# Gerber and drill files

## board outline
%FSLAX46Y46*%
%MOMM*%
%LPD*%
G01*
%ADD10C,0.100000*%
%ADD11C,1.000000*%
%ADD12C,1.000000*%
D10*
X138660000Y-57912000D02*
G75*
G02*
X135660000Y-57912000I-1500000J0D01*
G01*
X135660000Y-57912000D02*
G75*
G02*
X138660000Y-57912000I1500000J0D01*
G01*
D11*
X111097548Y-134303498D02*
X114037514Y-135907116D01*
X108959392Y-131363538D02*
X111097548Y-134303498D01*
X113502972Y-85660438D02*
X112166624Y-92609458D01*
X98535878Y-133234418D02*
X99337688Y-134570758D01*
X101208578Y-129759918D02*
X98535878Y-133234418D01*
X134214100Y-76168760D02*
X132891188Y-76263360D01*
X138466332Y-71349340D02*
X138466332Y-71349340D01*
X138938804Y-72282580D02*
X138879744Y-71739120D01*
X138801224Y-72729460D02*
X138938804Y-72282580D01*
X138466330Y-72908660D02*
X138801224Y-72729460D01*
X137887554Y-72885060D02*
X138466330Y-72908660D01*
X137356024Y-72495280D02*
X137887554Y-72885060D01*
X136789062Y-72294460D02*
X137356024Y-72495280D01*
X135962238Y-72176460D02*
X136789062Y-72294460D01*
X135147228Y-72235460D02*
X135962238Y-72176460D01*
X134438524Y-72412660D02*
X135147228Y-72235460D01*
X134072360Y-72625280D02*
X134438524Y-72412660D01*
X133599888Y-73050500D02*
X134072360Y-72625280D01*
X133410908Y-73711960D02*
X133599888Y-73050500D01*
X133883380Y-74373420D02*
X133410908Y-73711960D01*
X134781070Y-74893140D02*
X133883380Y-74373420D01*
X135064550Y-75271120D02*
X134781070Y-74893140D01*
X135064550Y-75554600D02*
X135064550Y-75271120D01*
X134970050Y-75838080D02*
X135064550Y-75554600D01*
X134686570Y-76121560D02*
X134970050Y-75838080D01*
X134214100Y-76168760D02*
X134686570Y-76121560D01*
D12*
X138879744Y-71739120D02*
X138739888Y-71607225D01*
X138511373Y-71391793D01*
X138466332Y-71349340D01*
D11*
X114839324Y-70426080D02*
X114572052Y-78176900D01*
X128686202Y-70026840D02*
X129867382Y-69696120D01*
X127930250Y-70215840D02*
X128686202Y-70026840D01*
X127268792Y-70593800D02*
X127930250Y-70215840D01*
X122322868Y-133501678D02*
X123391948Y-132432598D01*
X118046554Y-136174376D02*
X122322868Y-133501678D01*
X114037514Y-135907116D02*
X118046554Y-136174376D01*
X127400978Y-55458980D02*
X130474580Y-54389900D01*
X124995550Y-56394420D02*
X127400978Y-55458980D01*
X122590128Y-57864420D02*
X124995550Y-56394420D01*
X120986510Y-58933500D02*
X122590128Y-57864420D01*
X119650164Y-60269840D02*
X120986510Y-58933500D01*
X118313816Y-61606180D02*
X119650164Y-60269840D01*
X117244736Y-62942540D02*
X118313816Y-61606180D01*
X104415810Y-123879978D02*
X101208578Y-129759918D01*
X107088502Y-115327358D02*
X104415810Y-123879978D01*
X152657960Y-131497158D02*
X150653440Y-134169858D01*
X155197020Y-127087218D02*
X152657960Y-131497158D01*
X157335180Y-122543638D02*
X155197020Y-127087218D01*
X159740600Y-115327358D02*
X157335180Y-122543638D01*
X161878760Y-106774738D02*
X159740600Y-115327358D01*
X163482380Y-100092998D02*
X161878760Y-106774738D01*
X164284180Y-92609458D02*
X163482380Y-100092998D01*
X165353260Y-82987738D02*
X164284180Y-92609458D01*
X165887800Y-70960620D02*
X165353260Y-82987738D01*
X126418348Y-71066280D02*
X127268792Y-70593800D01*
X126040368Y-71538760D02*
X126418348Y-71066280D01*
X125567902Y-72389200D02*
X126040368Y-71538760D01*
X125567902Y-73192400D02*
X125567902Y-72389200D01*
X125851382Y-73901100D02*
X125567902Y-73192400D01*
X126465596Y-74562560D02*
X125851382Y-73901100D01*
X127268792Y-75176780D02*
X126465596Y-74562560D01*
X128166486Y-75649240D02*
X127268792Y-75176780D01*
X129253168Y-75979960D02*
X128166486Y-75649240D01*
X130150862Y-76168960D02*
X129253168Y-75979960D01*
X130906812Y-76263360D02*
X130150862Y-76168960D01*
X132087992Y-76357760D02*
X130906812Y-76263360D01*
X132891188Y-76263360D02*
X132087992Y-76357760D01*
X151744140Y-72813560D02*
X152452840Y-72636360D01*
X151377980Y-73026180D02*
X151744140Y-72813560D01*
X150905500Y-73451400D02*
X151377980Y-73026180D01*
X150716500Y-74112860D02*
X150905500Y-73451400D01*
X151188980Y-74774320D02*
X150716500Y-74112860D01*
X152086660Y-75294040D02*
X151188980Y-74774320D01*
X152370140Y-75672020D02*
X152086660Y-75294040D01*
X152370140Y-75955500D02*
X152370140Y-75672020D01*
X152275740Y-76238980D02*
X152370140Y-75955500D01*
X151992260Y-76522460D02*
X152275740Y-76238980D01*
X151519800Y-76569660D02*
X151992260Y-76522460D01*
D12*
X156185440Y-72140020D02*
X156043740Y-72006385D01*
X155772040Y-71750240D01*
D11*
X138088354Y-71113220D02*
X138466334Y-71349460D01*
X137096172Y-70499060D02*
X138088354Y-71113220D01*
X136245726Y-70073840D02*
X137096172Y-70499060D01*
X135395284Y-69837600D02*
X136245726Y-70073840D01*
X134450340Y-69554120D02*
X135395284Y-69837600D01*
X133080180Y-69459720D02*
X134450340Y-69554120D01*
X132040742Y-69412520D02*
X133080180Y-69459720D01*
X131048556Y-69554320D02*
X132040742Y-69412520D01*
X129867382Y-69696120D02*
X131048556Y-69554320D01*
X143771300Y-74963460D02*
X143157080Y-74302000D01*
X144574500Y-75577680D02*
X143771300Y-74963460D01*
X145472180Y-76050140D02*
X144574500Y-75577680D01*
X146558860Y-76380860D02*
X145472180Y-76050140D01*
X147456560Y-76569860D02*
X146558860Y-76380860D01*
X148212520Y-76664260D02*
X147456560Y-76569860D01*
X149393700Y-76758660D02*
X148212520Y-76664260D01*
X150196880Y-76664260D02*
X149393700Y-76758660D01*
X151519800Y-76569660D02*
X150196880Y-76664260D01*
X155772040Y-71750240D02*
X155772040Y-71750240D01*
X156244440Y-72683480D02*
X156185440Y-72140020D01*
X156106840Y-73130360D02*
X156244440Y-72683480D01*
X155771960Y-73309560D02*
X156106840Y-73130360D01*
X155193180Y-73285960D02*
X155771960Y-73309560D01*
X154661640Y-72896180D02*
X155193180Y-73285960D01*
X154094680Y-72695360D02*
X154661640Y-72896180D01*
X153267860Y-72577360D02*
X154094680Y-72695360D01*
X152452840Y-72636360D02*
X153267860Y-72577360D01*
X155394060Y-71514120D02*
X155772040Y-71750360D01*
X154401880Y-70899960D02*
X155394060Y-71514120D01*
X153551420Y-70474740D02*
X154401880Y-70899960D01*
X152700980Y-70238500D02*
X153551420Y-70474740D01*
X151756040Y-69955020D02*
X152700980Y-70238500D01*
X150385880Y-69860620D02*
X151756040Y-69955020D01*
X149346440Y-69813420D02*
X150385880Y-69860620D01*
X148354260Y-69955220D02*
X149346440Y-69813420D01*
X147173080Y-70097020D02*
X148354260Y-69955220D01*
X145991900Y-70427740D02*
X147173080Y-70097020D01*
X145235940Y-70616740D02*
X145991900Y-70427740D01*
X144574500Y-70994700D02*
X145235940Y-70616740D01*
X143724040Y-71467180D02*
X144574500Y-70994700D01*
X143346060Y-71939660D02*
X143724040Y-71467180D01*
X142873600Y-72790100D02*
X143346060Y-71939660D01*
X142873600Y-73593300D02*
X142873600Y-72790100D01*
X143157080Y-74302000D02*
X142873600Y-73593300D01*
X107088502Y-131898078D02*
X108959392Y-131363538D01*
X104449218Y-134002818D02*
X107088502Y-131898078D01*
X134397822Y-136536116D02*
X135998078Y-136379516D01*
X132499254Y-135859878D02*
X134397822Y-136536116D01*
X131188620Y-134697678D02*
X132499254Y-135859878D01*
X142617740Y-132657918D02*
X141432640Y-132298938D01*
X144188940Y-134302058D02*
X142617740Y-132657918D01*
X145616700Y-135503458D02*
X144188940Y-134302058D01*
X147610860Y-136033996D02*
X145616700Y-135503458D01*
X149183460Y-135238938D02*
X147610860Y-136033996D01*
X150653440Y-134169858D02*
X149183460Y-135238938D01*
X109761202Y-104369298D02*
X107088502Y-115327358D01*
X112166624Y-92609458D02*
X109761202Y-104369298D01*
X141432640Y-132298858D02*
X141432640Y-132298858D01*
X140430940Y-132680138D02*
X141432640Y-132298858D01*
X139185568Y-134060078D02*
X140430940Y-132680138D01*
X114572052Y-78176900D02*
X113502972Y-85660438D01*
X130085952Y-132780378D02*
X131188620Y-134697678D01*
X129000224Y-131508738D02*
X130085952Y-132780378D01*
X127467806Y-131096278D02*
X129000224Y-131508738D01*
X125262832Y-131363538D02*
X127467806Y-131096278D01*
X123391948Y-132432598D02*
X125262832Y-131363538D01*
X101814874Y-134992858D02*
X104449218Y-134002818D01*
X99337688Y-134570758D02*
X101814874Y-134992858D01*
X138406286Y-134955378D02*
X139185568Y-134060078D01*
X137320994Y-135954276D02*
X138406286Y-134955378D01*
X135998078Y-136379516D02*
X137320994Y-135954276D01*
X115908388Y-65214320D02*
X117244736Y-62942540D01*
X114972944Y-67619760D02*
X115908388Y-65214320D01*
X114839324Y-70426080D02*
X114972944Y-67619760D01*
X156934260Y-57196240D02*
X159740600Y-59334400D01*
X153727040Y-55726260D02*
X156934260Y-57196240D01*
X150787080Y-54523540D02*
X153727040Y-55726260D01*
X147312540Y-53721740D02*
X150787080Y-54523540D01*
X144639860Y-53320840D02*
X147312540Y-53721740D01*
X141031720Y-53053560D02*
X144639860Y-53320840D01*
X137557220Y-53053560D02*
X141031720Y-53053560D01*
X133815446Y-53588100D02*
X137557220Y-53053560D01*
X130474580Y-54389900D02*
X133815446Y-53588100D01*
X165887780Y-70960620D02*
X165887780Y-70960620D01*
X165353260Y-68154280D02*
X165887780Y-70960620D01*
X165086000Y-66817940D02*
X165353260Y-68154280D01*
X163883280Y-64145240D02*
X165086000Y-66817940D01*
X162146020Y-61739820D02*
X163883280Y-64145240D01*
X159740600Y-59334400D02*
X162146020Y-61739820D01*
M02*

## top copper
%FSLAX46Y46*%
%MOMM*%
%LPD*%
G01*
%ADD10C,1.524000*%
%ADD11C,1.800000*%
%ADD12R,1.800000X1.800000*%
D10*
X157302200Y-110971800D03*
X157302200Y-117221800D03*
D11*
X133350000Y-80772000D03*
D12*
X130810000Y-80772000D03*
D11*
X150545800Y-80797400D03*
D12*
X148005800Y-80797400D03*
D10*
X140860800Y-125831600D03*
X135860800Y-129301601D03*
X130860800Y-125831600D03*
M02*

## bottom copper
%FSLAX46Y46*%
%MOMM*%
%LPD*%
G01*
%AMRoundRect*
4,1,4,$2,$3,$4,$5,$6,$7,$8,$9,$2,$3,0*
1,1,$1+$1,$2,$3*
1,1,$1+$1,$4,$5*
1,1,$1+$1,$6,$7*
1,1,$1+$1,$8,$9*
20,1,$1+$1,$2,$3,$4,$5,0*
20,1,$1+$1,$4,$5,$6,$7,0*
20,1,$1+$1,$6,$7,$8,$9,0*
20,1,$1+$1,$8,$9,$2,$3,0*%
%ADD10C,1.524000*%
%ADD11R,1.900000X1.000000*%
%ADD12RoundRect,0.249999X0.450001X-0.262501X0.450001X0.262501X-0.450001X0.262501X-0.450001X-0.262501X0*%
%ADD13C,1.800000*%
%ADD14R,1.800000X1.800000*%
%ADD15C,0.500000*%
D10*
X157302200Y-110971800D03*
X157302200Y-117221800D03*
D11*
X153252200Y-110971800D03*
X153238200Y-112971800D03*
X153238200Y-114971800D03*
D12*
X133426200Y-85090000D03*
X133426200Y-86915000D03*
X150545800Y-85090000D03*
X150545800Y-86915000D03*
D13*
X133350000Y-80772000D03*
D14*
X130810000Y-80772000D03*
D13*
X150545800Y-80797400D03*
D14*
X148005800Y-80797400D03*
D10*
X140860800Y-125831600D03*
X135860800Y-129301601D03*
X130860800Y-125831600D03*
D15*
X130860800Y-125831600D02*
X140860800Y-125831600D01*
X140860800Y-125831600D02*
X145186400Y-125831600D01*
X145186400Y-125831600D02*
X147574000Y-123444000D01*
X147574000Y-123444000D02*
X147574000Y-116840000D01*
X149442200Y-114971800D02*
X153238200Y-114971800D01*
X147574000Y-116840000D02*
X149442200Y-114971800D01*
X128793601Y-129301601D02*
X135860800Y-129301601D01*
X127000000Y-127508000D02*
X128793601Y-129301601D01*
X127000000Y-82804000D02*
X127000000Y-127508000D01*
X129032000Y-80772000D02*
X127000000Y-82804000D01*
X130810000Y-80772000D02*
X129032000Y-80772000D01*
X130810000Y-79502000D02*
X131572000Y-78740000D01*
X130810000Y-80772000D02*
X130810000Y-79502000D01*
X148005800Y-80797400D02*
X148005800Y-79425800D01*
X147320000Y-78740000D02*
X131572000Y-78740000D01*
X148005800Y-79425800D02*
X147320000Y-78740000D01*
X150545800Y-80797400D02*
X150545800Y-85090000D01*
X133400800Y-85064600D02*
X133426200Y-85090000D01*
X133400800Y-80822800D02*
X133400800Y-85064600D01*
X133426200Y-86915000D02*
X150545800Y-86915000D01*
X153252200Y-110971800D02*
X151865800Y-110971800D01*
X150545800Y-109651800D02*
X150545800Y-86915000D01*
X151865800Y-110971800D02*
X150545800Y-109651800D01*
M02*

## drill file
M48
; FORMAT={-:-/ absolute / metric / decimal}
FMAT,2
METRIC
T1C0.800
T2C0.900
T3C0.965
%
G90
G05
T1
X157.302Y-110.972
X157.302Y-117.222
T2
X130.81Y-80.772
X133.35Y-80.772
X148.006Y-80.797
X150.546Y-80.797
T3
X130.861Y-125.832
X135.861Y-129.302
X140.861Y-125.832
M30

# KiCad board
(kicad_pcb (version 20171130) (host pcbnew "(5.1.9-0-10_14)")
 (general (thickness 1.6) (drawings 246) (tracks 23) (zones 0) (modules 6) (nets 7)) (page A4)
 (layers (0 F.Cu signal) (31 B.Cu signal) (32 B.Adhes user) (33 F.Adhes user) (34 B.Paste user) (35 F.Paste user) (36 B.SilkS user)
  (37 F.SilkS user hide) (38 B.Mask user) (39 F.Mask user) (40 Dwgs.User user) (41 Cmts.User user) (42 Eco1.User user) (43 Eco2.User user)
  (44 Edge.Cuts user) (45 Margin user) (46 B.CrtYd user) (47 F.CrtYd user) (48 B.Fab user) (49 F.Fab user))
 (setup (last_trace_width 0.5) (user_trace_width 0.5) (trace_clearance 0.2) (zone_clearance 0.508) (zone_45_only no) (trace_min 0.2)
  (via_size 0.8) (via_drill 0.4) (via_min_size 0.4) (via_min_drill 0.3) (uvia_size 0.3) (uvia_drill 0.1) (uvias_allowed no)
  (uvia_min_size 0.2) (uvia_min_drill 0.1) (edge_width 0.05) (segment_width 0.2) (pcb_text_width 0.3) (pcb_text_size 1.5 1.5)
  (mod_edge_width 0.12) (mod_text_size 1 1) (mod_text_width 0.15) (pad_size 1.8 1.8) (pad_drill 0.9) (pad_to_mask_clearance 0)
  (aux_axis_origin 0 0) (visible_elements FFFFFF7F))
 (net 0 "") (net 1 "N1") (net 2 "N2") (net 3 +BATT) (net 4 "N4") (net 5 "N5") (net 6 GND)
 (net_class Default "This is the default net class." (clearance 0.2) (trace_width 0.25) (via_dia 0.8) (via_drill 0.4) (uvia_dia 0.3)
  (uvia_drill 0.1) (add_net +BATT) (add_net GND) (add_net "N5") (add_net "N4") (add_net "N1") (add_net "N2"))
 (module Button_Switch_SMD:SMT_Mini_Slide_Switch (layer B.Cu) (at 155.0162 114.0968 270)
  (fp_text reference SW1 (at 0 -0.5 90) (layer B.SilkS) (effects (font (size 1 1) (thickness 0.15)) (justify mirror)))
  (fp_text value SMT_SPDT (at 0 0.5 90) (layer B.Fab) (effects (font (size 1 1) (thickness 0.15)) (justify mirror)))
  (pad "" thru_hole circle (at -3.125 -2.286 270) (size 1.524 1.524) (drill 0.8) (layers *.Cu *.Mask))
  (pad "" thru_hole circle (at 3.125 -2.286 270) (size 1.524 1.524) (drill 0.8) (layers *.Cu *.Mask))
  (pad 1 smd rect (at -3.125 1.764 270) (size 1 1.9) (layers B.Cu B.Paste B.Mask) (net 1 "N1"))
  (pad 2 smd rect (at -1.125 1.778 270) (size 1 1.9) (layers B.Cu B.Paste B.Mask) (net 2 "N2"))
  (pad 3 smd rect (at 0.875 1.778 270) (size 1 1.9) (layers B.Cu B.Paste B.Mask) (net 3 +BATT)))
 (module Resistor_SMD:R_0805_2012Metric (layer B.Cu) (at 133.4262 86.0025 90)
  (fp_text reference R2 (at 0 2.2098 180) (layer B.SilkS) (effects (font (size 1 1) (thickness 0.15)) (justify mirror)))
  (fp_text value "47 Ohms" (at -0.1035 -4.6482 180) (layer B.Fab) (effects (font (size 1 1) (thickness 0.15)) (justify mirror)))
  (pad 2 smd roundrect (at 0.9125 0 90) (size 1.025 1.4) (layers B.Cu B.Paste B.Mask) (roundrect_rratio 0.2439014634146341) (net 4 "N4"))
  (pad 1 smd roundrect (at -0.9125 0 90) (size 1.025 1.4) (layers B.Cu B.Paste B.Mask) (roundrect_rratio 0.2439014634146341) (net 1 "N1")))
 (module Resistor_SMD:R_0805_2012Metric (layer B.Cu) (at 150.5458 86.0025 90)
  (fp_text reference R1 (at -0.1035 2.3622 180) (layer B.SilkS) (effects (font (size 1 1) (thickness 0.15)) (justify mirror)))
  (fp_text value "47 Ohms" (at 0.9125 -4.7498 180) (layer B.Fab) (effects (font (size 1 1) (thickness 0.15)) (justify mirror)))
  (pad 2 smd roundrect (at 0.9125 0 90) (size 1.025 1.4) (layers B.Cu B.Paste B.Mask) (roundrect_rratio 0.2439014634146341) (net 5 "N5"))
  (pad 1 smd roundrect (at -0.9125 0 90) (size 1.025 1.4) (layers B.Cu B.Paste B.Mask) (roundrect_rratio 0.2439014634146341) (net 1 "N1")))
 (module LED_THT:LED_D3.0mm (layer B.Cu) (at 130.81 80.772)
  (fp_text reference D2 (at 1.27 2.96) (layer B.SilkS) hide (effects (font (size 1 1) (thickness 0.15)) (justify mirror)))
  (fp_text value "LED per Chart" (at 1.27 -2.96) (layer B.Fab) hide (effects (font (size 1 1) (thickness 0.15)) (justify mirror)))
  (pad 2 thru_hole circle (at 2.54 0) (size 1.8 1.8) (drill 0.9) (layers *.Cu *.Mask) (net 4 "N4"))
  (pad 1 thru_hole rect (at 0 0) (size 1.8 1.8) (drill 0.9) (layers *.Cu *.Mask) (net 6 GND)))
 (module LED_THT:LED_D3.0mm (layer B.Cu) (at 148.0058 80.7974)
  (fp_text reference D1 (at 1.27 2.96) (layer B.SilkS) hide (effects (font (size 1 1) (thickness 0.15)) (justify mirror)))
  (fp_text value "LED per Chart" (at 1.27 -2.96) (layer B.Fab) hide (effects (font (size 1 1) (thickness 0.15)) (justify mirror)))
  (pad 2 thru_hole circle (at 2.54 0) (size 1.8 1.8) (drill 0.9) (layers *.Cu *.Mask) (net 5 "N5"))
  (pad 1 thru_hole rect (at 0 0) (size 1.8 1.8) (drill 0.9) (layers *.Cu *.Mask) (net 6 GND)))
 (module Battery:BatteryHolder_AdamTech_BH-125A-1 (layer B.Cu) (at 130.8608 125.8316)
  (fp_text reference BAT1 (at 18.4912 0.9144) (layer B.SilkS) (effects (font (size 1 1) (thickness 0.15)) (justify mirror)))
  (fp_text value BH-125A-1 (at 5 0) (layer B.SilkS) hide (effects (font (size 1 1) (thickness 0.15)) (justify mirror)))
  (pad POS2 thru_hole circle (at 10 0) (size 1.524 1.524) (drill 0.9652) (layers *.Cu *.Mask) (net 3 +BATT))
  (pad NEG thru_hole circle (at 5 3.470001) (size 1.524 1.524) (drill 0.9652) (layers *.Cu *.Mask) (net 6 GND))
  (pad POS1 thru_hole circle (at 0 0) (size 1.524 1.524) (drill 0.9652) (layers *.Cu *.Mask) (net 3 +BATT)))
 (gr_circle (center 137.16 57.912) (end 138.66 57.912) (layer Edge.Cuts) (width 0.1))
 (gr_line (start 111.097548 134.303498) (end 114.037514 135.907116) (layer Edge.Cuts) (width 1))
 (gr_line (start 108.959392 131.363538) (end 111.097548 134.303498) (layer Edge.Cuts) (width 1))
 (gr_line (start 113.502972 85.660438) (end 112.166624 92.609458) (layer Edge.Cuts) (width 1))
 (gr_line (start 98.535878 133.234418) (end 99.337688 134.570758) (layer Edge.Cuts) (width 1))
 (gr_line (start 101.208578 129.759918) (end 98.535878 133.234418) (layer Edge.Cuts) (width 1))
 (gr_line (start 134.2141 76.16876) (end 132.891188 76.26336) (layer Edge.Cuts) (width 1))
 (gr_line (start 138.466332 71.34934) (end 138.466332 71.34934) (layer Edge.Cuts) (width 1))
 (gr_line (start 138.938804 72.28258) (end 138.879744 71.73912) (layer Edge.Cuts) (width 1))
 (gr_line (start 138.801224 72.72946) (end 138.938804 72.28258) (layer Edge.Cuts) (width 1))
 (gr_line (start 138.46633 72.90866) (end 138.801224 72.72946) (layer Edge.Cuts) (width 1))
 (gr_line (start 137.887554 72.88506) (end 138.46633 72.90866) (layer Edge.Cuts) (width 1))
 (gr_line (start 137.356024 72.49528) (end 137.887554 72.88506) (layer Edge.Cuts) (width 1))
 (gr_line (start 136.789062 72.29446) (end 137.356024 72.49528) (layer Edge.Cuts) (width 1))
 (gr_line (start 135.962238 72.17646) (end 136.789062 72.29446) (layer Edge.Cuts) (width 1))
 (gr_line (start 135.147228 72.23546) (end 135.962238 72.17646) (layer Edge.Cuts) (width 1))
 (gr_line (start 134.438524 72.41266) (end 135.147228 72.23546) (layer Edge.Cuts) (width 1))
 (gr_line (start 134.07236 72.62528) (end 134.438524 72.41266) (layer Edge.Cuts) (width 1))
 (gr_line (start 133.599888 73.0505) (end 134.07236 72.62528) (layer Edge.Cuts) (width 1))
 (gr_line (start 133.410908 73.71196) (end 133.599888 73.0505) (layer Edge.Cuts) (width 1))
 (gr_line (start 133.88338 74.37342) (end 133.410908 73.71196) (layer Edge.Cuts) (width 1))
 (gr_line (start 134.78107 74.89314) (end 133.88338 74.37342) (layer Edge.Cuts) (width 1))
 (gr_line (start 135.06455 75.27112) (end 134.78107 74.89314) (layer Edge.Cuts) (width 1))
 (gr_line (start 135.06455 75.5546) (end 135.06455 75.27112) (layer Edge.Cuts) (width 1))
 (gr_line (start 134.97005 75.83808) (end 135.06455 75.5546) (layer Edge.Cuts) (width 1))
 (gr_line (start 134.68657 76.12156) (end 134.97005 75.83808) (layer Edge.Cuts) (width 1))
 (gr_line (start 134.2141 76.16876) (end 134.68657 76.12156) (layer Edge.Cuts) (width 1))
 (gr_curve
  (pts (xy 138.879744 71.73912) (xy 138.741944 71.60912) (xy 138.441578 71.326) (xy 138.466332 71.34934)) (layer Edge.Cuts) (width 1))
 (gr_line (start 114.839324 70.42608) (end 114.572052 78.1769) (layer Edge.Cuts) (width 1))
 (gr_line (start 128.686202 70.02684) (end 129.867382 69.69612) (layer Edge.Cuts) (width 1))
 (gr_line (start 127.93025 70.21584) (end 128.686202 70.02684) (layer Edge.Cuts) (width 1))
 (gr_line (start 127.268792 70.5938) (end 127.93025 70.21584) (layer Edge.Cuts) (width 1))
 (gr_line (start 122.322868 133.501678) (end 123.391948 132.432598) (layer Edge.Cuts) (width 1))
 (gr_line (start 118.046554 136.174376) (end 122.322868 133.501678) (layer Edge.Cuts) (width 1))
 (gr_line (start 114.037514 135.907116) (end 118.046554 136.174376) (layer Edge.Cuts) (width 1))
 (gr_line (start 127.400978 55.45898) (end 130.47458 54.3899) (layer Edge.Cuts) (width 1))
 (gr_line (start 124.99555 56.39442) (end 127.400978 55.45898) (layer Edge.Cuts) (width 1))
 (gr_line (start 122.590128 57.86442) (end 124.99555 56.39442) (layer Edge.Cuts) (width 1))
 (gr_line (start 120.98651 58.9335) (end 122.590128 57.86442) (layer Edge.Cuts) (width 1))
 (gr_line (start 119.650164 60.26984) (end 120.98651 58.9335) (layer Edge.Cuts) (width 1))
 (gr_line (start 118.313816 61.60618) (end 119.650164 60.26984) (layer Edge.Cuts) (width 1))
 (gr_line (start 117.244736 62.94254) (end 118.313816 61.60618) (layer Edge.Cuts) (width 1))
 (gr_line (start 104.41581 123.879978) (end 101.208578 129.759918) (layer Edge.Cuts) (width 1))
 (gr_line (start 107.088502 115.327358) (end 104.41581 123.879978) (layer Edge.Cuts) (width 1))
 (gr_line (start 152.65796 131.497158) (end 150.65344 134.169858) (layer Edge.Cuts) (width 1))
 (gr_line (start 155.19702 127.087218) (end 152.65796 131.497158) (layer Edge.Cuts) (width 1))
 (gr_line (start 157.33518 122.543638) (end 155.19702 127.087218) (layer Edge.Cuts) (width 1))
 (gr_line (start 159.7406 115.327358) (end 157.33518 122.543638) (layer Edge.Cuts) (width 1))
 (gr_line (start 161.87876 106.774738) (end 159.7406 115.327358) (layer Edge.Cuts) (width 1))
 (gr_line (start 163.48238 100.092998) (end 161.87876 106.774738) (layer Edge.Cuts) (width 1))
 (gr_line (start 164.28418 92.609458) (end 163.48238 100.092998) (layer Edge.Cuts) (width 1))
 (gr_line (start 165.35326 82.987738) (end 164.28418 92.609458) (layer Edge.Cuts) (width 1))
 (gr_line (start 165.8878 70.96062) (end 165.35326 82.987738) (layer Edge.Cuts) (width 1))
 (gr_line (start 126.418348 71.06628) (end 127.268792 70.5938) (layer Edge.Cuts) (width 1))
 (gr_line (start 126.040368 71.53876) (end 126.418348 71.06628) (layer Edge.Cuts) (width 1))
 (gr_line (start 125.567902 72.3892) (end 126.040368 71.53876) (layer Edge.Cuts) (width 1))
 (gr_line (start 125.567902 73.1924) (end 125.567902 72.3892) (layer Edge.Cuts) (width 1))
 (gr_line (start 125.851382 73.9011) (end 125.567902 73.1924) (layer Edge.Cuts) (width 1))
 (gr_line (start 126.465596 74.56256) (end 125.851382 73.9011) (layer Edge.Cuts) (width 1))
 (gr_line (start 127.268792 75.17678) (end 126.465596 74.56256) (layer Edge.Cuts) (width 1))
 (gr_line (start 128.166486 75.64924) (end 127.268792 75.17678) (layer Edge.Cuts) (width 1))
 (gr_line (start 129.253168 75.97996) (end 128.166486 75.64924) (layer Edge.Cuts) (width 1))
 (gr_line (start 130.150862 76.16896) (end 129.253168 75.97996) (layer Edge.Cuts) (width 1))
 (gr_line (start 130.906812 76.26336) (end 130.150862 76.16896) (layer Edge.Cuts) (width 1))
 (gr_line (start 132.087992 76.35776) (end 130.906812 76.26336) (layer Edge.Cuts) (width 1))
 (gr_line (start 132.891188 76.26336) (end 132.087992 76.35776) (layer Edge.Cuts) (width 1))
 (gr_line (start 151.74414 72.81356) (end 152.45284 72.63636) (layer Edge.Cuts) (width 1))
 (gr_line (start 151.37798 73.02618) (end 151.74414 72.81356) (layer Edge.Cuts) (width 1))
 (gr_line (start 150.9055 73.4514) (end 151.37798 73.02618) (layer Edge.Cuts) (width 1))
 (gr_line (start 150.7165 74.11286) (end 150.9055 73.4514) (layer Edge.Cuts) (width 1))
 (gr_line (start 151.18898 74.77432) (end 150.7165 74.11286) (layer Edge.Cuts) (width 1))
 (gr_line (start 152.08666 75.29404) (end 151.18898 74.77432) (layer Edge.Cuts) (width 1))
 (gr_line (start 152.37014 75.67202) (end 152.08666 75.29404) (layer Edge.Cuts) (width 1))
 (gr_line (start 152.37014 75.9555) (end 152.37014 75.67202) (layer Edge.Cuts) (width 1))
 (gr_line (start 152.27574 76.23898) (end 152.37014 75.9555) (layer Edge.Cuts) (width 1))
 (gr_line (start 151.99226 76.52246) (end 152.27574 76.23898) (layer Edge.Cuts) (width 1))
 (gr_line (start 151.5198 76.56966) (end 151.99226 76.52246) (layer Edge.Cuts) (width 1))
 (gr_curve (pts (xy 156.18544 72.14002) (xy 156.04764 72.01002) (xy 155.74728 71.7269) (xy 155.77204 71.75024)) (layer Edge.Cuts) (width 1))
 (gr_line (start 138.088354 71.11322) (end 138.466334 71.34946) (layer Edge.Cuts) (width 1))
 (gr_line (start 137.096172 70.49906) (end 138.088354 71.11322) (layer Edge.Cuts) (width 1))
 (gr_line (start 136.245726 70.07384) (end 137.096172 70.49906) (layer Edge.Cuts) (width 1))
 (gr_line (start 135.395284 69.8376) (end 136.245726 70.07384) (layer Edge.Cuts) (width 1))
 (gr_line (start 134.45034 69.55412) (end 135.395284 69.8376) (layer Edge.Cuts) (width 1))
 (gr_line (start 133.08018 69.45972) (end 134.45034 69.55412) (layer Edge.Cuts) (width 1))
 (gr_line (start 132.040742 69.41252) (end 133.08018 69.45972) (layer Edge.Cuts) (width 1))
 (gr_line (start 131.048556 69.55432) (end 132.040742 69.41252) (layer Edge.Cuts) (width 1))
 (gr_line (start 129.867382 69.69612) (end 131.048556 69.55432) (layer Edge.Cuts) (width 1))
 (gr_line (start 143.7713 74.96346) (end 143.15708 74.302) (layer Edge.Cuts) (width 1))
 (gr_line (start 144.5745 75.57768) (end 143.7713 74.96346) (layer Edge.Cuts) (width 1))
 (gr_line (start 145.47218 76.05014) (end 144.5745 75.57768) (layer Edge.Cuts) (width 1))
 (gr_line (start 146.55886 76.38086) (end 145.47218 76.05014) (layer Edge.Cuts) (width 1))
 (gr_line (start 147.45656 76.56986) (end 146.55886 76.38086) (layer Edge.Cuts) (width 1))
 (gr_line (start 148.21252 76.66426) (end 147.45656 76.56986) (layer Edge.Cuts) (width 1))
 (gr_line (start 149.3937 76.75866) (end 148.21252 76.66426) (layer Edge.Cuts) (width 1))
 (gr_line (start 150.19688 76.66426) (end 149.3937 76.75866) (layer Edge.Cuts) (width 1))
 (gr_line (start 151.5198 76.56966) (end 150.19688 76.66426) (layer Edge.Cuts) (width 1))
 (gr_line (start 155.77204 71.75024) (end 155.77204 71.75024) (layer Edge.Cuts) (width 1))
 (gr_line (start 156.24444 72.68348) (end 156.18544 72.14002) (layer Edge.Cuts) (width 1))
 (gr_line (start 156.10684 73.13036) (end 156.24444 72.68348) (layer Edge.Cuts) (width 1))
 (gr_line (start 155.77196 73.30956) (end 156.10684 73.13036) (layer Edge.Cuts) (width 1))
 (gr_line (start 155.19318 73.28596) (end 155.77196 73.30956) (layer Edge.Cuts) (width 1))
 (gr_line (start 154.66164 72.89618) (end 155.19318 73.28596) (layer Edge.Cuts) (width 1))
 (gr_line (start 154.09468 72.69536) (end 154.66164 72.89618) (layer Edge.Cuts) (width 1))
 (gr_line (start 153.26786 72.57736) (end 154.09468 72.69536) (layer Edge.Cuts) (width 1))
 (gr_line (start 152.45284 72.63636) (end 153.26786 72.57736) (layer Edge.Cuts) (width 1))
 (gr_line (start 155.39406 71.51412) (end 155.77204 71.75036) (layer Edge.Cuts) (width 1))
 (gr_line (start 154.40188 70.89996) (end 155.39406 71.51412) (layer Edge.Cuts) (width 1))
 (gr_line (start 153.55142 70.47474) (end 154.40188 70.89996) (layer Edge.Cuts) (width 1))
 (gr_line (start 152.70098 70.2385) (end 153.55142 70.47474) (layer Edge.Cuts) (width 1))
 (gr_line (start 151.75604 69.95502) (end 152.70098 70.2385) (layer Edge.Cuts) (width 1))
 (gr_line (start 150.38588 69.86062) (end 151.75604 69.95502) (layer Edge.Cuts) (width 1))
 (gr_line (start 149.34644 69.81342) (end 150.38588 69.86062) (layer Edge.Cuts) (width 1))
 (gr_line (start 148.35426 69.95522) (end 149.34644 69.81342) (layer Edge.Cuts) (width 1))
 (gr_line (start 147.17308 70.09702) (end 148.35426 69.95522) (layer Edge.Cuts) (width 1))
 (gr_line (start 145.9919 70.42774) (end 147.17308 70.09702) (layer Edge.Cuts) (width 1))
 (gr_line (start 145.23594 70.61674) (end 145.9919 70.42774) (layer Edge.Cuts) (width 1))
 (gr_line (start 144.5745 70.9947) (end 145.23594 70.61674) (layer Edge.Cuts) (width 1))
 (gr_line (start 143.72404 71.46718) (end 144.5745 70.9947) (layer Edge.Cuts) (width 1))
 (gr_line (start 143.34606 71.93966) (end 143.72404 71.46718) (layer Edge.Cuts) (width 1))
 (gr_line (start 142.8736 72.7901) (end 143.34606 71.93966) (layer Edge.Cuts) (width 1))
 (gr_line (start 142.8736 73.5933) (end 142.8736 72.7901) (layer Edge.Cuts) (width 1))
 (gr_line (start 143.15708 74.302) (end 142.8736 73.5933) (layer Edge.Cuts) (width 1))
 (gr_line (start 107.088502 131.898078) (end 108.959392 131.363538) (layer Edge.Cuts) (width 1))
 (gr_line (start 104.449218 134.002818) (end 107.088502 131.898078) (layer Edge.Cuts) (width 1))
 (gr_line (start 134.397822 136.536116) (end 135.998078 136.379516) (layer Edge.Cuts) (width 1))
 (gr_line (start 132.499254 135.859878) (end 134.397822 136.536116) (layer Edge.Cuts) (width 1))
 (gr_line (start 131.18862 134.697678) (end 132.499254 135.859878) (layer Edge.Cuts) (width 1))
 (gr_line (start 142.61774 132.657918) (end 141.43264 132.298938) (layer Edge.Cuts) (width 1))
 (gr_line (start 144.18894 134.302058) (end 142.61774 132.657918) (layer Edge.Cuts) (width 1))
 (gr_line (start 145.6167 135.503458) (end 144.18894 134.302058) (layer Edge.Cuts) (width 1))
 (gr_line (start 147.61086 136.033996) (end 145.6167 135.503458) (layer Edge.Cuts) (width 1))
 (gr_line (start 149.18346 135.238938) (end 147.61086 136.033996) (layer Edge.Cuts) (width 1))
 (gr_line (start 150.65344 134.169858) (end 149.18346 135.238938) (layer Edge.Cuts) (width 1))
 (gr_line (start 109.761202 104.369298) (end 107.088502 115.327358) (layer Edge.Cuts) (width 1))
 (gr_line (start 112.166624 92.609458) (end 109.761202 104.369298) (layer Edge.Cuts) (width 1))
 (gr_line (start 141.43264 132.298858) (end 141.43264 132.298858) (layer Edge.Cuts) (width 1))
 (gr_line (start 140.43094 132.680138) (end 141.43264 132.298858) (layer Edge.Cuts) (width 1))
 (gr_line (start 139.185568 134.060078) (end 140.43094 132.680138) (layer Edge.Cuts) (width 1))
 (gr_line (start 114.572052 78.1769) (end 113.502972 85.660438) (layer Edge.Cuts) (width 1))
 (gr_line (start 130.085952 132.780378) (end 131.18862 134.697678) (layer Edge.Cuts) (width 1))
 (gr_line (start 129.000224 131.508738) (end 130.085952 132.780378) (layer Edge.Cuts) (width 1))
 (gr_line (start 127.467806 131.096278) (end 129.000224 131.508738) (layer Edge.Cuts) (width 1))
 (gr_line (start 125.262832 131.363538) (end 127.467806 131.096278) (layer Edge.Cuts) (width 1))
 (gr_line (start 123.391948 132.432598) (end 125.262832 131.363538) (layer Edge.Cuts) (width 1))
 (gr_line (start 101.814874 134.992858) (end 104.449218 134.002818) (layer Edge.Cuts) (width 1))
 (gr_line (start 99.337688 134.570758) (end 101.814874 134.992858) (layer Edge.Cuts) (width 1))
 (gr_line (start 138.406286 134.955378) (end 139.185568 134.060078) (layer Edge.Cuts) (width 1))
 (gr_line (start 137.320994 135.954276) (end 138.406286 134.955378) (layer Edge.Cuts) (width 1))
 (gr_line (start 135.998078 136.379516) (end 137.320994 135.954276) (layer Edge.Cuts) (width 1))
 (gr_line (start 115.908388 65.21432) (end 117.244736 62.94254) (layer Edge.Cuts) (width 1))
 (gr_line (start 114.972944 67.61976) (end 115.908388 65.21432) (layer Edge.Cuts) (width 1))
 (gr_line (start 114.839324 70.42608) (end 114.972944 67.61976) (layer Edge.Cuts) (width 1))
 (gr_line (start 156.93426 57.19624) (end 159.7406 59.3344) (layer Edge.Cuts) (width 1))
 (gr_line (start 153.72704 55.72626) (end 156.93426 57.19624) (layer Edge.Cuts) (width 1))
 (gr_line (start 150.78708 54.52354) (end 153.72704 55.72626) (layer Edge.Cuts) (width 1))
 (gr_line (start 147.31254 53.72174) (end 150.78708 54.52354) (layer Edge.Cuts) (width 1))
 (gr_line (start 144.63986 53.32084) (end 147.31254 53.72174) (layer Edge.Cuts) (width 1))
 (gr_line (start 141.03172 53.05356) (end 144.63986 53.32084) (layer Edge.Cuts) (width 1))
 (gr_line (start 137.55722 53.05356) (end 141.03172 53.05356) (layer Edge.Cuts) (width 1))
 (gr_line (start 133.815446 53.5881) (end 137.55722 53.05356) (layer Edge.Cuts) (width 1))
 (gr_line (start 130.47458 54.3899) (end 133.815446 53.5881) (layer Edge.Cuts) (width 1))
 (gr_line (start 165.88778 70.96062) (end 165.88778 70.96062) (layer Edge.Cuts) (width 1))
 (gr_line (start 165.35326 68.15428) (end 165.88778 70.96062) (layer Edge.Cuts) (width 1))
 (gr_line (start 165.086 66.81794) (end 165.35326 68.15428) (layer Edge.Cuts) (width 1))
 (gr_line (start 163.88328 64.14524) (end 165.086 66.81794) (layer Edge.Cuts) (width 1))
 (gr_line (start 162.14602 61.73982) (end 163.88328 64.14524) (layer Edge.Cuts) (width 1))
 (gr_line (start 159.7406 59.3344) (end 162.14602 61.73982) (layer Edge.Cuts) (width 1))
 (segment (start 130.8608 125.8316) (end 140.8608 125.8316) (width 0.5) (layer B.Cu) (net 3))
 (segment (start 140.8608 125.8316) (end 145.1864 125.8316) (width 0.5) (layer B.Cu) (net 3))
 (segment (start 145.1864 125.8316) (end 147.574 123.444) (width 0.5) (layer B.Cu) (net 3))
 (segment (start 147.574 123.444) (end 147.574 116.84) (width 0.5) (layer B.Cu) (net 3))
 (segment (start 149.4422 114.9718) (end 153.2382 114.9718) (width 0.5) (layer B.Cu) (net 3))
 (segment (start 147.574 116.84) (end 149.4422 114.9718) (width 0.5) (layer B.Cu) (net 3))
 (segment (start 128.793601 129.301601) (end 135.8608 129.301601) (width 0.5) (layer B.Cu) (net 6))
 (segment (start 127 127.508) (end 128.793601 129.301601) (width 0.5) (layer B.Cu) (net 6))
 (segment (start 127 82.804) (end 127 127.508) (width 0.5) (layer B.Cu) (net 6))
 (segment (start 129.032 80.772) (end 127 82.804) (width 0.5) (layer B.Cu) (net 6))
 (segment (start 130.81 80.772) (end 129.032 80.772) (width 0.5) (layer B.Cu) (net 6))
 (segment (start 130.81 79.502) (end 131.572 78.74) (width 0.5) (layer B.Cu) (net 6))
 (segment (start 130.81 80.772) (end 130.81 79.502) (width 0.5) (layer B.Cu) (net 6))
 (segment (start 148.0058 80.7974) (end 148.0058 79.4258) (width 0.5) (layer B.Cu) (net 6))
 (segment (start 147.32 78.74) (end 131.572 78.74) (width 0.5) (layer B.Cu) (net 6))
 (segment (start 148.0058 79.4258) (end 147.32 78.74) (width 0.5) (layer B.Cu) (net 6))
 (segment (start 150.5458 80.7974) (end 150.5458 85.09) (width 0.5) (layer B.Cu) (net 5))
 (segment (start 133.4008 85.0646) (end 133.4262 85.09) (width 0.5) (layer B.Cu) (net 4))
 (segment (start 133.4008 80.8228) (end 133.4008 85.0646) (width 0.5) (layer B.Cu) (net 4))
 (segment (start 133.4262 86.915) (end 150.5458 86.915) (width 0.5) (layer B.Cu) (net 1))
 (segment (start 153.2522 110.9718) (end 151.8658 110.9718) (width 0.5) (layer B.Cu) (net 1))
 (segment (start 150.5458 109.6518) (end 150.5458 86.915) (width 0.5) (layer B.Cu) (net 1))
 (segment (start 151.8658 110.9718) (end 150.5458 109.6518) (width 0.5) (layer B.Cu) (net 1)))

